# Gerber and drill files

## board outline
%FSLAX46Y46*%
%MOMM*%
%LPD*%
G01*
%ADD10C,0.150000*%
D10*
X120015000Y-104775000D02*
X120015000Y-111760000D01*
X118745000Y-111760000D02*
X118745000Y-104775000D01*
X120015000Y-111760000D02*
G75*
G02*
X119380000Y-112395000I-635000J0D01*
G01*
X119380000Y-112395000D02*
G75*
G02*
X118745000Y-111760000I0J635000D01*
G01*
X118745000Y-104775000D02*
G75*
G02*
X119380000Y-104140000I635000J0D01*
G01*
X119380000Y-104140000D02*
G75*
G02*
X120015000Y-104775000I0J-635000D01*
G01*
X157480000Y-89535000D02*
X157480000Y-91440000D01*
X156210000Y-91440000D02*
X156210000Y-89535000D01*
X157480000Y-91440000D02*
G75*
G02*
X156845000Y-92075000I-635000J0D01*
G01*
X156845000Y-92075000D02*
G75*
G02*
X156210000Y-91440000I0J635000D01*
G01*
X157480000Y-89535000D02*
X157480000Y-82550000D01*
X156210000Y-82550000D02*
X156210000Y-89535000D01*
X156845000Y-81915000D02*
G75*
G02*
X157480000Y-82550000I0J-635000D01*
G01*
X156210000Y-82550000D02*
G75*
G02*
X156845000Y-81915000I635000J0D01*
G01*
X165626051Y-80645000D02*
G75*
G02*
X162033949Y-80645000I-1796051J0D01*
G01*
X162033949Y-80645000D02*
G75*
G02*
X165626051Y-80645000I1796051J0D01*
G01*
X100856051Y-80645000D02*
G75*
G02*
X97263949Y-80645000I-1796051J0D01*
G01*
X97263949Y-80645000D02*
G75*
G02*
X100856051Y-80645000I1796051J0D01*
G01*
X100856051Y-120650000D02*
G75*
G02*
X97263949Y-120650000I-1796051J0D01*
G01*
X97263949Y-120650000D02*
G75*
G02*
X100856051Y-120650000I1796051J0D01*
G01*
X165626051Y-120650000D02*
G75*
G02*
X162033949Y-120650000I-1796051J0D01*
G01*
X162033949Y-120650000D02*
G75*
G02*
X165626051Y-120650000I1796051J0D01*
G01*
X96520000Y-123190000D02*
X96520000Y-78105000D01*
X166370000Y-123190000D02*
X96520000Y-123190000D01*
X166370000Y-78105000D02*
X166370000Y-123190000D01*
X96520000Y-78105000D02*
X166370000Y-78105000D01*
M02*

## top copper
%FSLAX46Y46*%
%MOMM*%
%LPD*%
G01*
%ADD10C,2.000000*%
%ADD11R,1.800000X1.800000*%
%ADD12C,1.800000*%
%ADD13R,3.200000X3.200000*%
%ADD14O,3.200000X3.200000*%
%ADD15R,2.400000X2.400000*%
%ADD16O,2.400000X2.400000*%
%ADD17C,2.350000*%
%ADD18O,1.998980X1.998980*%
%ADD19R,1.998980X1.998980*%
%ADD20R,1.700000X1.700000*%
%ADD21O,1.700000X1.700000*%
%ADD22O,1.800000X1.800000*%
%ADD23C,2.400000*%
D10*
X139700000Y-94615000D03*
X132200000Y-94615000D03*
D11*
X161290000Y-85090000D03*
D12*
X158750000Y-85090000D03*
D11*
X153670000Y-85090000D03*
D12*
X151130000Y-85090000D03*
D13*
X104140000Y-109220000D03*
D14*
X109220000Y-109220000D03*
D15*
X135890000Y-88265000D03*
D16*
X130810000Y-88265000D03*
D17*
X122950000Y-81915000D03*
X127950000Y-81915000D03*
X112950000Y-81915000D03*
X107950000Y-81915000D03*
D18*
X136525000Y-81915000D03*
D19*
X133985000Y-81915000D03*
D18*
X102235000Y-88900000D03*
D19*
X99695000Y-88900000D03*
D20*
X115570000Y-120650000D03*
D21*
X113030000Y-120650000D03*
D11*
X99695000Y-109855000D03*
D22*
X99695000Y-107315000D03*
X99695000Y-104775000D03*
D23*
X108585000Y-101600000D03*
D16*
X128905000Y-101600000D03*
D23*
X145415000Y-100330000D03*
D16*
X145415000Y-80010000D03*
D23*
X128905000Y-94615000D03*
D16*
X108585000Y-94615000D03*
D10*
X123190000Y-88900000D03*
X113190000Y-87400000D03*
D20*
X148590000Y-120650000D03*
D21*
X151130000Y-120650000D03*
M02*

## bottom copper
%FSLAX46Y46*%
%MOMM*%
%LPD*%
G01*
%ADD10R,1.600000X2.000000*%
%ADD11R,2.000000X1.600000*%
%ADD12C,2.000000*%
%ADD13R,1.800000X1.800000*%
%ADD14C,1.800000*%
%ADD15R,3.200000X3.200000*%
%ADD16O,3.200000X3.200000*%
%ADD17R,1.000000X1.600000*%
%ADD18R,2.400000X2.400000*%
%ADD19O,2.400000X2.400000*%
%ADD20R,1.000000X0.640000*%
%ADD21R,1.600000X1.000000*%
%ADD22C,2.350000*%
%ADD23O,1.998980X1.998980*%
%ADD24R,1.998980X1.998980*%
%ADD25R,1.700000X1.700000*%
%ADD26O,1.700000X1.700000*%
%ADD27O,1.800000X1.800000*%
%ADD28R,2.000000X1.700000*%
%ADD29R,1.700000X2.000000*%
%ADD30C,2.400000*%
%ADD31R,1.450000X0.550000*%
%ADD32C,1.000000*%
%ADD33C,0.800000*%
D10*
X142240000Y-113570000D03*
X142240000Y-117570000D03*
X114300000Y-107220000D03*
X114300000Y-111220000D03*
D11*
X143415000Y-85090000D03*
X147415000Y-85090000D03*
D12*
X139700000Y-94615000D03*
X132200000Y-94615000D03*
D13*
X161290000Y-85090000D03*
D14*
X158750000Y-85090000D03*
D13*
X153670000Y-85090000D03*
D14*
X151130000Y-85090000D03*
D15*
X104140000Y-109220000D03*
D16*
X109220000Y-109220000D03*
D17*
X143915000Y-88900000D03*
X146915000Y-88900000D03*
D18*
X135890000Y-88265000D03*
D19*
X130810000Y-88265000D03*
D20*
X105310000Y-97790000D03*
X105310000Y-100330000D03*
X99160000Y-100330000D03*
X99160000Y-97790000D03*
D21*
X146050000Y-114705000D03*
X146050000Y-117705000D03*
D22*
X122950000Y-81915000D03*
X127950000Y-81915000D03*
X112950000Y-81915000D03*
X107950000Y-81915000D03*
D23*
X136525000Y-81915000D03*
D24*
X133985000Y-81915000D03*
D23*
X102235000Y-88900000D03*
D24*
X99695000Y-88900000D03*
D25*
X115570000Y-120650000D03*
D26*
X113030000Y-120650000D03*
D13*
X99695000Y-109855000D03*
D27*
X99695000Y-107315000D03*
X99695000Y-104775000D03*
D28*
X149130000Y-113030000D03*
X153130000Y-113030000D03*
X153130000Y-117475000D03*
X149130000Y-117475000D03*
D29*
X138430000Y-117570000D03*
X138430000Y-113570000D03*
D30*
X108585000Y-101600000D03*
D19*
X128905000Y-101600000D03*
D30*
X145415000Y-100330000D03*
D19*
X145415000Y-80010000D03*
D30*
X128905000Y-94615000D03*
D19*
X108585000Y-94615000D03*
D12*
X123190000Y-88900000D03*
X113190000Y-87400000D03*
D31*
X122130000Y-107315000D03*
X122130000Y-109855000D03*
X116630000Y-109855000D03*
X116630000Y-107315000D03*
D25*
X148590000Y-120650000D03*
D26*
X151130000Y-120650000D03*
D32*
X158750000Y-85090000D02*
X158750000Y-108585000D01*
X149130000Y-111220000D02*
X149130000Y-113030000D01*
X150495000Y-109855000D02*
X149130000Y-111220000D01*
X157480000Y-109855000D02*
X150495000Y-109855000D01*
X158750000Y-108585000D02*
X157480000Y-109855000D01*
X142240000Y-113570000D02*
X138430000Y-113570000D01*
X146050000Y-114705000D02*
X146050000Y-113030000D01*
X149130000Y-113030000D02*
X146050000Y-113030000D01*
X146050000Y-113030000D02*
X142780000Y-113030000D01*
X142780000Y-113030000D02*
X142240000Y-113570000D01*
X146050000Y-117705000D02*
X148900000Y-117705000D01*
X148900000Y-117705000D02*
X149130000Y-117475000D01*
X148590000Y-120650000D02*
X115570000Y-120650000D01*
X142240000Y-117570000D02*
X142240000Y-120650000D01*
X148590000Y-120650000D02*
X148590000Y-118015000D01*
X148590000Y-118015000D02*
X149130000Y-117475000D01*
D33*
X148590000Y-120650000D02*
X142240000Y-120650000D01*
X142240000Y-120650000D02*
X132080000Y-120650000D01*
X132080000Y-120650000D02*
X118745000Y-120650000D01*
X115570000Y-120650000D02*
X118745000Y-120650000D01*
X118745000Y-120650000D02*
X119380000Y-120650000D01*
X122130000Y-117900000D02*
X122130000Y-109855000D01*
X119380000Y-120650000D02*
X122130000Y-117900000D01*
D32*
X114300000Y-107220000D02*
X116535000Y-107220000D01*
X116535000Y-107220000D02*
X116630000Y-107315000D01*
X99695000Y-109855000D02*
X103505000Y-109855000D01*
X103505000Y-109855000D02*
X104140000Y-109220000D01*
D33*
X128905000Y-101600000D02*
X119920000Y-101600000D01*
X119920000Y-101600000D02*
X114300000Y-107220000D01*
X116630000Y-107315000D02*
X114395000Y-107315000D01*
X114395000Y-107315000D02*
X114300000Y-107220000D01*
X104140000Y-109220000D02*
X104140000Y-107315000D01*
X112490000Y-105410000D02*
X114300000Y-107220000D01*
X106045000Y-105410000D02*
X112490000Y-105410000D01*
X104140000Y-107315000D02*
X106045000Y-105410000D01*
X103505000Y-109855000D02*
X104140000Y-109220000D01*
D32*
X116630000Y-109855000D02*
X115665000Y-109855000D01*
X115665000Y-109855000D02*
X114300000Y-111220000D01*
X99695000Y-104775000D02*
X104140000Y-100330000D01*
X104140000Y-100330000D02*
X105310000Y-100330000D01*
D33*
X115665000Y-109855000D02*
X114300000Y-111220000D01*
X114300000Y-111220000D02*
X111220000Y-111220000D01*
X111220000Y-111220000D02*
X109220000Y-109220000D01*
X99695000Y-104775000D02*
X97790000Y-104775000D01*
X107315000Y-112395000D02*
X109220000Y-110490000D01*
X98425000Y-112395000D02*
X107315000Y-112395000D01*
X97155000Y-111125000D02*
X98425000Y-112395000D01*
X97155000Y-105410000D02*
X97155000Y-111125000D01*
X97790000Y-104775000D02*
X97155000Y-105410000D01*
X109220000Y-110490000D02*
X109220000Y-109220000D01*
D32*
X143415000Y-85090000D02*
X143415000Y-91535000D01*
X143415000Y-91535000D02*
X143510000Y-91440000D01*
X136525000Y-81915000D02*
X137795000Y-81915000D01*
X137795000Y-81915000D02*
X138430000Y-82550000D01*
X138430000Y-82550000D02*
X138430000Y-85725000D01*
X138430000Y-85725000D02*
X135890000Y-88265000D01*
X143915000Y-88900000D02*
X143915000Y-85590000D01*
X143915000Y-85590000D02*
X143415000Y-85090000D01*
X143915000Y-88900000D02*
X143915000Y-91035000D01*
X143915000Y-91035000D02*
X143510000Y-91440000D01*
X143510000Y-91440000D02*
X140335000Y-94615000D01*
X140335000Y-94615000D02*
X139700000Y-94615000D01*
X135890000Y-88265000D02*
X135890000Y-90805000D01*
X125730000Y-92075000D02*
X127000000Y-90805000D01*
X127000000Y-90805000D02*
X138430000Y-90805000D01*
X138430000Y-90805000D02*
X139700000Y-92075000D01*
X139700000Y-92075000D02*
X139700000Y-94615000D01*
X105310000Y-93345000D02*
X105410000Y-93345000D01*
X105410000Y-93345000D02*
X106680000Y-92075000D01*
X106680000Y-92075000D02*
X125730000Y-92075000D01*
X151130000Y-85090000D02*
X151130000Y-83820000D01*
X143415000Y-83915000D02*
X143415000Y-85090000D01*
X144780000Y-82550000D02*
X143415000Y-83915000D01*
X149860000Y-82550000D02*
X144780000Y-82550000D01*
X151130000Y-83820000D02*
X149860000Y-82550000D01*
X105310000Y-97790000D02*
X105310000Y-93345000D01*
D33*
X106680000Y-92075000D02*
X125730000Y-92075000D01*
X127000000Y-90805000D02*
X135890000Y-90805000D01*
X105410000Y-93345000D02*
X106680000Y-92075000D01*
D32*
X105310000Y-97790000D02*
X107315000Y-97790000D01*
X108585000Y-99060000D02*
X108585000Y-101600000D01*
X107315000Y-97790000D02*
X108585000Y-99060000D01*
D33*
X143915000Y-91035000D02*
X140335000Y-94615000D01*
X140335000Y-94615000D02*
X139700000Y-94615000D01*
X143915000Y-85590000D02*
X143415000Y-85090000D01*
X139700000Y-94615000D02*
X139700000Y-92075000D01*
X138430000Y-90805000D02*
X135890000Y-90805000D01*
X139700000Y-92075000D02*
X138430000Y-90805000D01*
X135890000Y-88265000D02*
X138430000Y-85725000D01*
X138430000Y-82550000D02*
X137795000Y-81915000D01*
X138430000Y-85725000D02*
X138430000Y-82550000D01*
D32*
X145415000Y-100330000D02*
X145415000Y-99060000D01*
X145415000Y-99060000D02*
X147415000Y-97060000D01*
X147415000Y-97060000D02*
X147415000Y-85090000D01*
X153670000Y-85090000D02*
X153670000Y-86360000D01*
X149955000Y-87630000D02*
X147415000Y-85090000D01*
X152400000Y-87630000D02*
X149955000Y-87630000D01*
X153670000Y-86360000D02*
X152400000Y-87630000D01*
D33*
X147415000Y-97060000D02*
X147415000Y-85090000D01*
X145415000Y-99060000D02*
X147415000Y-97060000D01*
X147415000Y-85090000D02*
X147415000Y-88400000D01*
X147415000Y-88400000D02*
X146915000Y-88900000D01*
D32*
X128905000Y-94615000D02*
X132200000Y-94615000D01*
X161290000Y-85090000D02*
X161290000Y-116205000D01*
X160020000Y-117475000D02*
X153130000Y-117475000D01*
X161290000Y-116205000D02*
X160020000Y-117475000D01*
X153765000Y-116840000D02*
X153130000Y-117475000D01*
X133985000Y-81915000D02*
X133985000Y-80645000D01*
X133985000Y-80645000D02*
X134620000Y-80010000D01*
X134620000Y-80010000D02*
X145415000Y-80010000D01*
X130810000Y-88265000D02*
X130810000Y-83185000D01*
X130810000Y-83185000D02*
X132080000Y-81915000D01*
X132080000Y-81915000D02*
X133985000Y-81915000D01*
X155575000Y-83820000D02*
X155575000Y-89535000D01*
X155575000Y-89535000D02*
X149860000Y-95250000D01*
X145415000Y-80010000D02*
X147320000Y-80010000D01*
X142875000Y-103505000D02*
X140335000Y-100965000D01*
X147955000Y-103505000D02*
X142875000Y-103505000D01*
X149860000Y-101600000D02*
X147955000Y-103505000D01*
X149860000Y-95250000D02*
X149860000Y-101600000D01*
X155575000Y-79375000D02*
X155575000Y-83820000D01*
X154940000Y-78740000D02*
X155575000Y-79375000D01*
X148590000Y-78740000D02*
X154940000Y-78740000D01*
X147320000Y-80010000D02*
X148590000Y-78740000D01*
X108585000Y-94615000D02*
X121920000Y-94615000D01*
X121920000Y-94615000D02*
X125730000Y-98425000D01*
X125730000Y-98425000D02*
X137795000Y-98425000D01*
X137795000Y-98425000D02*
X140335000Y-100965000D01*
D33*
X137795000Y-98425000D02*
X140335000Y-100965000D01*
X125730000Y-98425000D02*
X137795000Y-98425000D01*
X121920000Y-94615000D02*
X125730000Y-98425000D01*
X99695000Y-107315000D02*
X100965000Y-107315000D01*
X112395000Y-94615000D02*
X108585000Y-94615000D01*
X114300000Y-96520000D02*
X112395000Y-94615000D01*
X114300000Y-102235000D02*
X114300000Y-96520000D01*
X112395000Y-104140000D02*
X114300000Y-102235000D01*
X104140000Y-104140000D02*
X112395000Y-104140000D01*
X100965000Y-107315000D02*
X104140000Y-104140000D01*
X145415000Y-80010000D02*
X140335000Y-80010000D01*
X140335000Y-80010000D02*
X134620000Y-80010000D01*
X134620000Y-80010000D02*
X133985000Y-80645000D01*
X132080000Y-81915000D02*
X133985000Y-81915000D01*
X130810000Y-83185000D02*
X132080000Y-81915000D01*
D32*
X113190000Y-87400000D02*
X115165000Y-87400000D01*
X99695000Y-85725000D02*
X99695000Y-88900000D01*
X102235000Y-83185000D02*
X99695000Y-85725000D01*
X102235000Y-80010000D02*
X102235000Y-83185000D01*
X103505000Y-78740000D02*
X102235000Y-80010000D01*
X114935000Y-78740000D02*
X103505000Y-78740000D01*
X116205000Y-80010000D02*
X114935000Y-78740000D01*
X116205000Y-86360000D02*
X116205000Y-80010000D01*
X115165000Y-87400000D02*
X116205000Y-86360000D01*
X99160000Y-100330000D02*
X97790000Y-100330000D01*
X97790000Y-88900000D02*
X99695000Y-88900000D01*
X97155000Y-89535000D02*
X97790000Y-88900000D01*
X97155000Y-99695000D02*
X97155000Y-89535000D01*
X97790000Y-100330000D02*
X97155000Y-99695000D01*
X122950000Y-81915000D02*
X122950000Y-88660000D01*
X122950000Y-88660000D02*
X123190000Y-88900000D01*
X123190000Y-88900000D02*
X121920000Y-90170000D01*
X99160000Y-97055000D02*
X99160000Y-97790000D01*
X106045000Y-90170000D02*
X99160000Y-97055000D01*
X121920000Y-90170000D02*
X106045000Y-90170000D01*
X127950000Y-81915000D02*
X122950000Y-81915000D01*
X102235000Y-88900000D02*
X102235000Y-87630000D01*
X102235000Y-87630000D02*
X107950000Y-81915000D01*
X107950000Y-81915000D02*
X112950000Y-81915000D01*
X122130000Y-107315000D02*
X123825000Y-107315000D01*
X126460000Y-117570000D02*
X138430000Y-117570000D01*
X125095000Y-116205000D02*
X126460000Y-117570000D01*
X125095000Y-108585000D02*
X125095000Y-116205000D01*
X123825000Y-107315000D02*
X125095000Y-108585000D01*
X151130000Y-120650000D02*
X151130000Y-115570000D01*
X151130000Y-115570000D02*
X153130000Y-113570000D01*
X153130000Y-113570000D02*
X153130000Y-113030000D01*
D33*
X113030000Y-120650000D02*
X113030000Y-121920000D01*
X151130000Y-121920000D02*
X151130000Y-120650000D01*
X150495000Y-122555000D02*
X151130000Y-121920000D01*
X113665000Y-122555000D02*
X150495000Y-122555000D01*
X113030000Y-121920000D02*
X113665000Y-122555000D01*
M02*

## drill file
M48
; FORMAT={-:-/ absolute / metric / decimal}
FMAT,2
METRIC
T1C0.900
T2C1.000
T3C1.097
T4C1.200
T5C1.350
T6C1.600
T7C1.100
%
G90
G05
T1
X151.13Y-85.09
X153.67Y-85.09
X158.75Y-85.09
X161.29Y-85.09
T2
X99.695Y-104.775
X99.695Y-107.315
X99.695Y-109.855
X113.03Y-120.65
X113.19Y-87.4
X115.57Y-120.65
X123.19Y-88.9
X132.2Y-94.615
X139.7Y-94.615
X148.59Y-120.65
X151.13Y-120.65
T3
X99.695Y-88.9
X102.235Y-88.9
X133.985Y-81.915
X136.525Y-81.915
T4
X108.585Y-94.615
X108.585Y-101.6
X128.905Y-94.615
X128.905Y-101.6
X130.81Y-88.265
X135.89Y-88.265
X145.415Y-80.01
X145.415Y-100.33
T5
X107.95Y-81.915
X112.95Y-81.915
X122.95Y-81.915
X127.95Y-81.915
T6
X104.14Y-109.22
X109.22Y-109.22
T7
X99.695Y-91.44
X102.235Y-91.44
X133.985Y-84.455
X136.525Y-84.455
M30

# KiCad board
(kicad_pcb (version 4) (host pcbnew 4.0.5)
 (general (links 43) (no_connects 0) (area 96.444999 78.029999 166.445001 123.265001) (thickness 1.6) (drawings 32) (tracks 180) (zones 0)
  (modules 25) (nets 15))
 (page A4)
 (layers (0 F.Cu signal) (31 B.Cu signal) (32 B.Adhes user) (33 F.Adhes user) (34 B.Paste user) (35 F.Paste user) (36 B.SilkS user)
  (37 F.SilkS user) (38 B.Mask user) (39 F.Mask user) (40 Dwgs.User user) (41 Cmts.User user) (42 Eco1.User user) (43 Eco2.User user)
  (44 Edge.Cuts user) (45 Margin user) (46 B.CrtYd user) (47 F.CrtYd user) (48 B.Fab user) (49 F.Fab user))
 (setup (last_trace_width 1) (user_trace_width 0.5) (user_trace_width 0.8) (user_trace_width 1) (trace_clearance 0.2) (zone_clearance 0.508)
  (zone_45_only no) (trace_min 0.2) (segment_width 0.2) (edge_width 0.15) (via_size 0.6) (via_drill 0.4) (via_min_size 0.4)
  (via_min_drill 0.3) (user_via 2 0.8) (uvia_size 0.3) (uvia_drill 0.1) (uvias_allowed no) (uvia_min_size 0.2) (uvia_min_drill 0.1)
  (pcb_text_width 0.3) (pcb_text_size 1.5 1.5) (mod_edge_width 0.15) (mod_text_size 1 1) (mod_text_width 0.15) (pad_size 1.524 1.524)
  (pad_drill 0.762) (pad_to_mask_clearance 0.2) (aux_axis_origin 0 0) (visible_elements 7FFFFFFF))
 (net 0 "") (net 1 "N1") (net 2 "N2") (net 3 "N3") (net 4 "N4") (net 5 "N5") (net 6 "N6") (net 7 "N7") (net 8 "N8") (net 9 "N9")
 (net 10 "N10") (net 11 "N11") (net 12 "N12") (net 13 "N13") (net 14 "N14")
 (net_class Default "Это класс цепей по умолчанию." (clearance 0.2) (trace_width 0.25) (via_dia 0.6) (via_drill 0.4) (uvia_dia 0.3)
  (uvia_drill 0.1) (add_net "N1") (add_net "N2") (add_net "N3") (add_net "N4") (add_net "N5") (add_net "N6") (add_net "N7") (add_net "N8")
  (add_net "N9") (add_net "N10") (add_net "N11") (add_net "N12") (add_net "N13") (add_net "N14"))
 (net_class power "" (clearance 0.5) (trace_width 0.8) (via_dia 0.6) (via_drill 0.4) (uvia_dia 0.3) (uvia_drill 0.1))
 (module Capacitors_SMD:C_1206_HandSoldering (layer B.Cu) (at 142.24 115.57 270)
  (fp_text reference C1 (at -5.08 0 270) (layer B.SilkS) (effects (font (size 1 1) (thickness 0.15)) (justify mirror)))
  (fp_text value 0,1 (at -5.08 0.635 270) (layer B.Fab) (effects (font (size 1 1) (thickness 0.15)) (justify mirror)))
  (pad 1 smd rect (at -2 0 270) (size 2 1.6) (layers B.Cu B.Paste B.Mask) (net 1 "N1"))
  (pad 2 smd rect (at 2 0 270) (size 2 1.6) (layers B.Cu B.Paste B.Mask) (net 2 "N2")))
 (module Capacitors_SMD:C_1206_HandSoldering (layer B.Cu) (at 114.3 109.22 270)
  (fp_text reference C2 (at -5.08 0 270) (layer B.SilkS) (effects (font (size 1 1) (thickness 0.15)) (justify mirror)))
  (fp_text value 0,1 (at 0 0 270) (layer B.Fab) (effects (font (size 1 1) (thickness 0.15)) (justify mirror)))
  (pad 1 smd rect (at -2 0 270) (size 2 1.6) (layers B.Cu B.Paste B.Mask) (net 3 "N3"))
  (pad 2 smd rect (at 2 0 270) (size 2 1.6) (layers B.Cu B.Paste B.Mask) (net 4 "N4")))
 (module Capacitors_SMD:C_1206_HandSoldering (layer B.Cu) (at 145.415 85.09)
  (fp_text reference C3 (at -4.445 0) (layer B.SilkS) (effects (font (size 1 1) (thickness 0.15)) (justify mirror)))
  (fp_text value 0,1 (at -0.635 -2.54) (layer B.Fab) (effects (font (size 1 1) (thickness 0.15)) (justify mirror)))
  (pad 1 smd rect (at -2 0) (size 2 1.6) (layers B.Cu B.Paste B.Mask) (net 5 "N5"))
  (pad 2 smd rect (at 2 0) (size 2 1.6) (layers B.Cu B.Paste B.Mask) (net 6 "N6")))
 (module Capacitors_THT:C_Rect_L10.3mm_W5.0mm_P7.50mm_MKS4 (layer F.Cu) (at 139.7 94.615 180)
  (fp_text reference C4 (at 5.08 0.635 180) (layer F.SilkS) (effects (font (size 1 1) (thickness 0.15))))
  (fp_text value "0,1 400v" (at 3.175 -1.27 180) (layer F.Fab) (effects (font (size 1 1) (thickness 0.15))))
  (pad 1 thru_hole circle (at 0 0 180) (size 2 2) (drill 1) (layers *.Cu *.Mask) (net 5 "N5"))
  (pad 2 thru_hole circle (at 7.5 0 180) (size 2 2) (drill 1) (layers *.Cu *.Mask) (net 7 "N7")))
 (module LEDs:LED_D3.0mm (layer F.Cu) (at 161.29 85.09 180)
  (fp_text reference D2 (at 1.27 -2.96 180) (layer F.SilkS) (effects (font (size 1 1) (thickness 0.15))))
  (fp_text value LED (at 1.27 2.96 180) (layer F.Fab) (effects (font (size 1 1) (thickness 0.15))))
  (pad 1 thru_hole rect (at 0 0 180) (size 1.8 1.8) (drill 0.9) (layers *.Cu *.Mask) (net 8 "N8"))
  (pad 2 thru_hole circle (at 2.54 0 180) (size 1.8 1.8) (drill 0.9) (layers *.Cu *.Mask) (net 1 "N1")))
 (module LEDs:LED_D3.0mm (layer F.Cu) (at 153.67 85.09 180)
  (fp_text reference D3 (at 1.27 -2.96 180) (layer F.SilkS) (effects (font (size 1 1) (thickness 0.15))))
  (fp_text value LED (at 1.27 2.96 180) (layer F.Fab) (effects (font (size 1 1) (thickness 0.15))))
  (pad 1 thru_hole rect (at 0 0 180) (size 1.8 1.8) (drill 0.9) (layers *.Cu *.Mask) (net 6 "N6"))
  (pad 2 thru_hole circle (at 2.54 0 180) (size 1.8 1.8) (drill 0.9) (layers *.Cu *.Mask) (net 5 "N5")))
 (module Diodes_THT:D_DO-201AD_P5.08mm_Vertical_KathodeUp (layer F.Cu) (at 104.14 109.22)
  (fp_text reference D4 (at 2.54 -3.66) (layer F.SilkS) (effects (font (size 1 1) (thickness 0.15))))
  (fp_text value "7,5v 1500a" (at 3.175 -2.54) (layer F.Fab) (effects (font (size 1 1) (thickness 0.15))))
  (pad 1 thru_hole rect (at 0 0) (size 3.2 3.2) (drill 1.6) (layers *.Cu *.Mask) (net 3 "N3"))
  (pad 2 thru_hole oval (at 5.08 0) (size 3.2 3.2) (drill 1.6) (layers *.Cu *.Mask) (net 4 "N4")))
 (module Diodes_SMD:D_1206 (layer B.Cu) (at 145.415 88.9)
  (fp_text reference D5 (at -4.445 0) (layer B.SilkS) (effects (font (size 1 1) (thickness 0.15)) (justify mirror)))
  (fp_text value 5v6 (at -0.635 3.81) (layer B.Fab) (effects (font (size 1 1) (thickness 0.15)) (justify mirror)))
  (pad 1 smd rect (at -1.5 0) (size 1 1.6) (layers B.Cu B.Paste B.Mask) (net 5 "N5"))
  (pad 2 smd rect (at 1.5 0) (size 1 1.6) (layers B.Cu B.Paste B.Mask) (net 6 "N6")))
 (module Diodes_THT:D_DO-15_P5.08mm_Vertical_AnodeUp (layer F.Cu) (at 135.89 88.265 180)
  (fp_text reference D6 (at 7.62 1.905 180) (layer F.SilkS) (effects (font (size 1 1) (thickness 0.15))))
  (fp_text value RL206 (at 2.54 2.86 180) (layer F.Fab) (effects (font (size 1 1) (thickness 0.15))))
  (pad 1 thru_hole rect (at 0 0 180) (size 2.4 2.4) (drill 1.2) (layers *.Cu *.Mask) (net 5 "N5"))
  (pad 2 thru_hole oval (at 5.08 0 180) (size 2.4 2.4) (drill 1.2) (layers *.Cu *.Mask) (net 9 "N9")))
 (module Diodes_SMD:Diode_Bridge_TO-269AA (layer B.Cu) (at 102.235 99.06 180)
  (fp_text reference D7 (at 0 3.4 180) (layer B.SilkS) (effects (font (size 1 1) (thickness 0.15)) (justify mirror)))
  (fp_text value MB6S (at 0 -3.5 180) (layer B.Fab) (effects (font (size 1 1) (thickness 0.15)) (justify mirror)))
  (pad 1 smd rect (at -3.075 1.27 180) (size 1 0.64) (layers B.Cu B.Paste B.Mask) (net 5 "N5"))
  (pad 2 smd rect (at -3.075 -1.27 180) (size 1 0.64) (layers B.Cu B.Paste B.Mask) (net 4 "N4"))
  (pad 3 smd rect (at 3.075 -1.27 180) (size 1 0.64) (layers B.Cu B.Paste B.Mask) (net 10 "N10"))
  (pad 4 smd rect (at 3.075 1.27 180) (size 1 0.64) (layers B.Cu B.Paste B.Mask) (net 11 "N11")))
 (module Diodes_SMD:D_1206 (layer B.Cu) (at 146.05 116.205 270)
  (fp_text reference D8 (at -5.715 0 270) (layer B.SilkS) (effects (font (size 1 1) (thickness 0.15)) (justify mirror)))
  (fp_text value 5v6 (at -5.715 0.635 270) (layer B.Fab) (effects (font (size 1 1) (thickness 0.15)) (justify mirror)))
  (pad 1 smd rect (at -1.5 0 270) (size 1 1.6) (layers B.Cu B.Paste B.Mask) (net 1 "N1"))
  (pad 2 smd rect (at 1.5 0 270) (size 1 1.6) (layers B.Cu B.Paste B.Mask) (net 2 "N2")))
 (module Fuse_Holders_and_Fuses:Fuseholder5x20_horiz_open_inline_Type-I (layer F.Cu) (at 107.95 81.915)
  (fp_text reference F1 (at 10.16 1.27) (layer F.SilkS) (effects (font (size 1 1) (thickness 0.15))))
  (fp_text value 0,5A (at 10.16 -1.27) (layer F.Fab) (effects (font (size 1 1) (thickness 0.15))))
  (pad 2 thru_hole circle (at 15 0) (size 2.35 2.35) (drill 1.35) (layers *.Cu *.Mask) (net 11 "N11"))
  (pad 2 thru_hole circle (at 20 0) (size 2.35 2.35) (drill 1.35) (layers *.Cu *.Mask) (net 11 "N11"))
  (pad 1 thru_hole circle (at 5 0) (size 2.35 2.35) (drill 1.35) (layers *.Cu *.Mask) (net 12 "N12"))
  (pad 1 thru_hole circle (at 0 0) (size 2.35 2.35) (drill 1.35) (layers *.Cu *.Mask) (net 12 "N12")))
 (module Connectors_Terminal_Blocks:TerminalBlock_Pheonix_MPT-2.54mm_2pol (layer F.Cu) (at 133.985 81.915)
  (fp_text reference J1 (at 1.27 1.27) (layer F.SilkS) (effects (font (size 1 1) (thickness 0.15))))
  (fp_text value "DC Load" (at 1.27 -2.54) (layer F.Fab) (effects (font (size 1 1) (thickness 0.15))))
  (pad 2 thru_hole oval (at 2.54 0) (size 1.99898 1.99898) (drill 1.09728) (layers *.Cu *.Mask) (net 5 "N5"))
  (pad 1 thru_hole rect (at 0 0) (size 1.99898 1.99898) (drill 1.09728) (layers *.Cu *.Mask) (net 9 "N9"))
  (pad "" np_thru_hole circle (at 0 2.54) (size 1.1 1.1) (drill 1.1) (layers *.Cu *.Mask))
  (pad "" np_thru_hole circle (at 2.54 2.54) (size 1.1 1.1) (drill 1.1) (layers *.Cu *.Mask)))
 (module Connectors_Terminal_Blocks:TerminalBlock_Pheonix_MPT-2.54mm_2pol (layer F.Cu) (at 99.695 88.9)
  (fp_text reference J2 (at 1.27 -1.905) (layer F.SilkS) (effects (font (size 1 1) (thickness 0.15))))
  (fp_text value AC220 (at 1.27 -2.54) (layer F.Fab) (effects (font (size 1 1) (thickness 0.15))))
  (pad 2 thru_hole oval (at 2.54 0) (size 1.99898 1.99898) (drill 1.09728) (layers *.Cu *.Mask) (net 12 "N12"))
  (pad 1 thru_hole rect (at 0 0) (size 1.99898 1.99898) (drill 1.09728) (layers *.Cu *.Mask) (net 10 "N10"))
  (pad "" np_thru_hole circle (at 0 2.54) (size 1.1 1.1) (drill 1.1) (layers *.Cu *.Mask))
  (pad "" np_thru_hole circle (at 2.54 2.54) (size 1.1 1.1) (drill 1.1) (layers *.Cu *.Mask)))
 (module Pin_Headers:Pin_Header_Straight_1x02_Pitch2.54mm (layer F.Cu) (at 115.57 120.65 270)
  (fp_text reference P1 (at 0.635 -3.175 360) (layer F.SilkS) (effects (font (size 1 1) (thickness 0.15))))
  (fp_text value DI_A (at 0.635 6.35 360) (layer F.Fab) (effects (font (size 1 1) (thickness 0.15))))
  (pad 1 thru_hole rect (at 0 0 270) (size 1.7 1.7) (drill 1) (layers *.Cu *.Mask) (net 2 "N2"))
  (pad 2 thru_hole oval (at 0 2.54 270) (size 1.7 1.7) (drill 1) (layers *.Cu *.Mask) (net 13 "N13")))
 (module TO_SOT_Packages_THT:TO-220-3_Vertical (layer F.Cu) (at 99.695 109.855 90)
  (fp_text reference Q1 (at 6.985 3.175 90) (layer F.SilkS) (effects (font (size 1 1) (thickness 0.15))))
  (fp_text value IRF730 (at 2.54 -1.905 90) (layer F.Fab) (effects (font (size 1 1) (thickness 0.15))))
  (pad 1 thru_hole rect (at 0 0 90) (size 1.8 1.8) (drill 1) (layers *.Cu *.Mask) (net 3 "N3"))
  (pad 2 thru_hole oval (at 2.54 0 90) (size 1.8 1.8) (drill 1) (layers *.Cu *.Mask) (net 9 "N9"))
  (pad 3 thru_hole oval (at 5.08 0 90) (size 1.8 1.8) (drill 1) (layers *.Cu *.Mask) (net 4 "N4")))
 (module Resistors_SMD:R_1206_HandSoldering (layer B.Cu) (at 151.13 113.03)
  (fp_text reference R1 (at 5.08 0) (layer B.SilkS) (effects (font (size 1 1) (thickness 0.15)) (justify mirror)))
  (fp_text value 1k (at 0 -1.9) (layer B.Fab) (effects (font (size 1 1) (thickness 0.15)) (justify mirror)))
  (pad 1 smd rect (at -2 0) (size 2 1.7) (layers B.Cu B.Paste B.Mask) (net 1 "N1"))
  (pad 2 smd rect (at 2 0) (size 2 1.7) (layers B.Cu B.Paste B.Mask) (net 13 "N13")))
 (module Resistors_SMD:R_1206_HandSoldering (layer B.Cu) (at 151.13 117.475 180)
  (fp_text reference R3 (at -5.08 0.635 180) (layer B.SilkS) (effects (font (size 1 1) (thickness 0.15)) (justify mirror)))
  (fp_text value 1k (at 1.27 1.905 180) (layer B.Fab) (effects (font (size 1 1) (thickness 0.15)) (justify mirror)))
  (pad 1 smd rect (at -2 0 180) (size 2 1.7) (layers B.Cu B.Paste B.Mask) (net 8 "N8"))
  (pad 2 smd rect (at 2 0 180) (size 2 1.7) (layers B.Cu B.Paste B.Mask) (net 2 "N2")))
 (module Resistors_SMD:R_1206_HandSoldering (layer B.Cu) (at 138.43 115.57 90)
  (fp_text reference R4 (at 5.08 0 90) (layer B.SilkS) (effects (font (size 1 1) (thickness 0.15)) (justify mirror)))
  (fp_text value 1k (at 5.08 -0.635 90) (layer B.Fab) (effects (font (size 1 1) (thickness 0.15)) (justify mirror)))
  (pad 1 smd rect (at -2 0 90) (size 2 1.7) (layers B.Cu B.Paste B.Mask) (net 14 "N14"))
  (pad 2 smd rect (at 2 0 90) (size 2 1.7) (layers B.Cu B.Paste B.Mask) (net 1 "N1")))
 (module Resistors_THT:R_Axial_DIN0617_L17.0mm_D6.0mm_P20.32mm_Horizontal (layer F.Cu) (at 108.585 101.6)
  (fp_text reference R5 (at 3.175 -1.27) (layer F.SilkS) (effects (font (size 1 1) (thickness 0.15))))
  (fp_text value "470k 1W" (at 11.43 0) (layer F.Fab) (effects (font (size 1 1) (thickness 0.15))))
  (pad 1 thru_hole circle (at 0 0) (size 2.4 2.4) (drill 1.2) (layers *.Cu *.Mask) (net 5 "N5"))
  (pad 2 thru_hole oval (at 20.32 0) (size 2.4 2.4) (drill 1.2) (layers *.Cu *.Mask) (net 3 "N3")))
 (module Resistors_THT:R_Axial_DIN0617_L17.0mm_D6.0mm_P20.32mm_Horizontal (layer F.Cu) (at 145.415 100.33 90)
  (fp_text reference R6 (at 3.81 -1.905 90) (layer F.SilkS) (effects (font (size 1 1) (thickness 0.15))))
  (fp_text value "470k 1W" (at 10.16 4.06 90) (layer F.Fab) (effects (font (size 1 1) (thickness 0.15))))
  (pad 1 thru_hole circle (at 0 0 90) (size 2.4 2.4) (drill 1.2) (layers *.Cu *.Mask) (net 6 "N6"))
  (pad 2 thru_hole oval (at 20.32 0 90) (size 2.4 2.4) (drill 1.2) (layers *.Cu *.Mask) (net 9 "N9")))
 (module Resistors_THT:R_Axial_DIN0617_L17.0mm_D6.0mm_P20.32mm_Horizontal (layer F.Cu) (at 128.905 94.615 180)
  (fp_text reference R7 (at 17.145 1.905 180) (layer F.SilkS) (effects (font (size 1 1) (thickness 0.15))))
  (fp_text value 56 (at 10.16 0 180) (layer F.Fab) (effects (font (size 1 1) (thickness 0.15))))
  (pad 1 thru_hole circle (at 0 0 180) (size 2.4 2.4) (drill 1.2) (layers *.Cu *.Mask) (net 7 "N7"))
  (pad 2 thru_hole oval (at 20.32 0 180) (size 2.4 2.4) (drill 1.2) (layers *.Cu *.Mask) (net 9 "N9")))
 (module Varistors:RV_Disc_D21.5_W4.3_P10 (layer F.Cu) (at 123.19 88.9 180)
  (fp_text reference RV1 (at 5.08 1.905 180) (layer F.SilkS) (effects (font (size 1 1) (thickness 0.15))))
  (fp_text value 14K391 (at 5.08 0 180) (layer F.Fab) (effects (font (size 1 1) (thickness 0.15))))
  (pad 1 thru_hole circle (at 0 0 180) (size 2 2) (drill 1) (layers *.Cu *.Mask) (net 11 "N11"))
  (pad 2 thru_hole circle (at 10 1.5 180) (size 2 2) (drill 1) (layers *.Cu *.Mask) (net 10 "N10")))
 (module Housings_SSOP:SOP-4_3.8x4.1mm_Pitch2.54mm (layer B.Cu) (at 119.38 108.585 180)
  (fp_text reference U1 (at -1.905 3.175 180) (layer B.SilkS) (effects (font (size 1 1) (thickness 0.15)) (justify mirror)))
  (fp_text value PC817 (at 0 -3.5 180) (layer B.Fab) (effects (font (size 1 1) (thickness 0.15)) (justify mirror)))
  (pad 1 smd rect (at -2.75 1.27 180) (size 1.45 0.55) (layers B.Cu B.Paste B.Mask) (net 14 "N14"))
  (pad 2 smd rect (at -2.75 -1.27 180) (size 1.45 0.55) (layers B.Cu B.Paste B.Mask) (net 2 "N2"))
  (pad 3 smd rect (at 2.75 -1.27 180) (size 1.45 0.55) (layers B.Cu B.Paste B.Mask) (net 4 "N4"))
  (pad 4 smd rect (at 2.75 1.27 180) (size 1.45 0.55) (layers B.Cu B.Paste B.Mask) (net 3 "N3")))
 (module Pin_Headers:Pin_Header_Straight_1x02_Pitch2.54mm (layer F.Cu) (at 148.59 120.65 90)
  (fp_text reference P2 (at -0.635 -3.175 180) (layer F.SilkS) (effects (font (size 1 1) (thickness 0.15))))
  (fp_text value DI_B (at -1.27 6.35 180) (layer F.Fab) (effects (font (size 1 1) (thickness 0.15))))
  (pad 1 thru_hole rect (at 0 0 90) (size 1.7 1.7) (drill 1) (layers *.Cu *.Mask) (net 2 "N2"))
  (pad 2 thru_hole oval (at 0 2.54 90) (size 1.7 1.7) (drill 1) (layers *.Cu *.Mask) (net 13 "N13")))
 (gr_line (start 120.015 104.775) (end 120.015 111.76) (angle 90) (layer Edge.Cuts) (width 0.15))
 (gr_line (start 118.745 111.76) (end 118.745 104.775) (angle 90) (layer Edge.Cuts) (width 0.15))
 (gr_arc (start 119.38 111.76) (end 120.015 111.76) (angle 90) (layer Edge.Cuts) (width 0.15))
 (gr_arc (start 119.38 111.76) (end 119.38 112.395) (angle 90) (layer Edge.Cuts) (width 0.15))
 (gr_arc (start 119.38 104.775) (end 118.745 104.775) (angle 90) (layer Edge.Cuts) (width 0.15))
 (gr_arc (start 119.38 104.775) (end 119.38 104.14) (angle 90) (layer Edge.Cuts) (width 0.15))
 (gr_line (start 157.48 89.535) (end 157.48 91.44) (angle 90) (layer Edge.Cuts) (width 0.15))
 (gr_line (start 156.21 91.44) (end 156.21 89.535) (angle 90) (layer Edge.Cuts) (width 0.15))
 (gr_arc (start 156.845 91.44) (end 157.48 91.44) (angle 90) (layer Edge.Cuts) (width 0.15))
 (gr_arc (start 156.845 91.44) (end 156.845 92.075) (angle 90) (layer Edge.Cuts) (width 0.15))
 (gr_line (start 157.48 89.535) (end 157.48 82.55) (angle 90) (layer Edge.Cuts) (width 0.15))
 (gr_line (start 156.21 82.55) (end 156.21 89.535) (angle 90) (layer Edge.Cuts) (width 0.15))
 (gr_arc (start 156.845 82.55) (end 156.845 81.915) (angle 90) (layer Edge.Cuts) (width 0.15))
 (gr_arc (start 156.845 82.55) (end 156.21 82.55) (angle 90) (layer Edge.Cuts) (width 0.15))
 (gr_circle (center 163.83 80.645) (end 165.1 79.375) (layer Edge.Cuts) (width 0.15))
 (gr_circle (center 99.06 80.645) (end 97.79 79.375) (layer Edge.Cuts) (width 0.15))
 (gr_circle (center 99.06 120.65) (end 97.79 121.92) (layer Edge.Cuts) (width 0.15))
 (gr_circle (center 163.83 120.65) (end 165.1 121.92) (layer Edge.Cuts) (width 0.15))
 (gr_line (start 96.52 123.19) (end 96.52 78.105) (angle 90) (layer Edge.Cuts) (width 0.15))
 (gr_line (start 166.37 123.19) (end 96.52 123.19) (angle 90) (layer Edge.Cuts) (width 0.15))
 (gr_line (start 166.37 78.105) (end 166.37 123.19) (angle 90) (layer Edge.Cuts) (width 0.15))
 (gr_line (start 96.52 78.105) (end 166.37 78.105) (angle 90) (layer Edge.Cuts) (width 0.15))
 (segment (start 158.75 85.09) (end 158.75 108.585) (width 1) (layer B.Cu) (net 1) (status 400000))
 (segment (start 149.13 111.22) (end 149.13 113.03) (width 1) (layer B.Cu) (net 1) (status 800000))
 (segment (start 150.495 109.855) (end 149.13 111.22) (width 1) (layer B.Cu) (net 1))
 (segment (start 157.48 109.855) (end 150.495 109.855) (width 1) (layer B.Cu) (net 1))
 (segment (start 158.75 108.585) (end 157.48 109.855) (width 1) (layer B.Cu) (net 1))
 (segment (start 142.24 113.57) (end 138.43 113.57) (width 1) (layer B.Cu) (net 1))
 (segment (start 146.05 114.705) (end 146.05 113.03) (width 1) (layer B.Cu) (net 1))
 (segment (start 149.13 113.03) (end 146.05 113.03) (width 1) (layer B.Cu) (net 1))
 (segment (start 146.05 113.03) (end 142.78 113.03) (width 1) (layer B.Cu) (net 1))
 (segment (start 142.78 113.03) (end 142.24 113.57) (width 1) (layer B.Cu) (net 1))
 (segment (start 146.05 117.705) (end 148.9 117.705) (width 1) (layer B.Cu) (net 2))
 (segment (start 148.9 117.705) (end 149.13 117.475) (width 1) (layer B.Cu) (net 2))
 (segment (start 148.59 120.65) (end 115.57 120.65) (width 1) (layer B.Cu) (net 2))
 (segment (start 142.24 117.57) (end 142.24 120.65) (width 1) (layer B.Cu) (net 2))
 (segment (start 148.59 120.65) (end 148.59 118.015) (width 1) (layer B.Cu) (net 2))
 (segment (start 148.59 118.015) (end 149.13 117.475) (width 1) (layer B.Cu) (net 2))
 (segment (start 148.59 120.65) (end 142.24 120.65) (width 0.8) (layer B.Cu) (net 2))
 (segment (start 142.24 120.65) (end 132.08 120.65) (width 0.8) (layer B.Cu) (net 2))
 (segment (start 132.08 120.65) (end 118.745 120.65) (width 0.8) (layer B.Cu) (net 2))
 (segment (start 115.57 120.65) (end 118.745 120.65) (width 0.8) (layer B.Cu) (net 2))
 (segment (start 118.745 120.65) (end 119.38 120.65) (width 0.8) (layer B.Cu) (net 2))
 (segment (start 122.13 117.9) (end 122.13 109.855) (width 0.8) (layer B.Cu) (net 2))
 (segment (start 119.38 120.65) (end 122.13 117.9) (width 0.8) (layer B.Cu) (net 2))
 (segment (start 114.3 107.22) (end 116.535 107.22) (width 1) (layer B.Cu) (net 3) (status C00000))
 (segment (start 116.535 107.22) (end 116.63 107.315) (width 1) (layer B.Cu) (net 3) (status C00000))
 (segment (start 99.695 109.855) (end 103.505 109.855) (width 1) (layer B.Cu) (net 3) (status C00000))
 (segment (start 103.505 109.855) (end 104.14 109.22) (width 1) (layer B.Cu) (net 3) (status C00000))
 (segment (start 128.905 101.6) (end 119.92 101.6) (width 0.8) (layer B.Cu) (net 3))
 (segment (start 119.92 101.6) (end 114.3 107.22) (width 0.8) (layer B.Cu) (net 3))
 (segment (start 116.63 107.315) (end 114.395 107.315) (width 0.8) (layer B.Cu) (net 3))
 (segment (start 114.395 107.315) (end 114.3 107.22) (width 0.8) (layer B.Cu) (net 3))
 (segment (start 104.14 109.22) (end 104.14 107.315) (width 0.8) (layer B.Cu) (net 3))
 (segment (start 112.49 105.41) (end 114.3 107.22) (width 0.8) (layer B.Cu) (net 3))
 (segment (start 106.045 105.41) (end 112.49 105.41) (width 0.8) (layer B.Cu) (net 3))
 (segment (start 104.14 107.315) (end 106.045 105.41) (width 0.8) (layer B.Cu) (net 3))
 (segment (start 103.505 109.855) (end 104.14 109.22) (width 0.8) (layer B.Cu) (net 3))
 (segment (start 116.63 109.855) (end 115.665 109.855) (width 1) (layer B.Cu) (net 4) (status 400000))
 (segment (start 115.665 109.855) (end 114.3 111.22) (width 1) (layer B.Cu) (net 4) (status 800000))
 (segment (start 99.695 104.775) (end 104.14 100.33) (width 1) (layer B.Cu) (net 4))
 (segment (start 104.14 100.33) (end 105.31 100.33) (width 1) (layer B.Cu) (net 4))
 (segment (start 115.665 109.855) (end 114.3 111.22) (width 0.8) (layer B.Cu) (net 4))
 (segment (start 114.3 111.22) (end 111.22 111.22) (width 0.8) (layer B.Cu) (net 4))
 (segment (start 111.22 111.22) (end 109.22 109.22) (width 0.8) (layer B.Cu) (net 4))
 (segment (start 99.695 104.775) (end 97.79 104.775) (width 0.8) (layer B.Cu) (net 4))
 (segment (start 107.315 112.395) (end 109.22 110.49) (width 0.8) (layer B.Cu) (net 4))
 (segment (start 98.425 112.395) (end 107.315 112.395) (width 0.8) (layer B.Cu) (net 4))
 (segment (start 97.155 111.125) (end 98.425 112.395) (width 0.8) (layer B.Cu) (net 4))
 (segment (start 97.155 105.41) (end 97.155 111.125) (width 0.8) (layer B.Cu) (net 4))
 (segment (start 97.79 104.775) (end 97.155 105.41) (width 0.8) (layer B.Cu) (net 4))
 (segment (start 109.22 110.49) (end 109.22 109.22) (width 0.8) (layer B.Cu) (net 4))
 (segment (start 143.415 85.09) (end 143.415 91.535) (width 1) (layer B.Cu) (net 5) (status 400000))
 (segment (start 143.415 91.535) (end 143.51 91.44) (width 1) (layer B.Cu) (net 5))
 (segment (start 136.525 81.915) (end 137.795 81.915) (width 1) (layer B.Cu) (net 5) (status 400000))
 (segment (start 137.795 81.915) (end 138.43 82.55) (width 1) (layer B.Cu) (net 5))
 (segment (start 138.43 82.55) (end 138.43 85.725) (width 1) (layer B.Cu) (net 5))
 (segment (start 138.43 85.725) (end 135.89 88.265) (width 1) (layer B.Cu) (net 5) (status 800000))
 (segment (start 143.915 88.9) (end 143.915 85.59) (width 1) (layer B.Cu) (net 5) (status C00000))
 (segment (start 143.915 85.59) (end 143.415 85.09) (width 1) (layer B.Cu) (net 5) (status C00000))
 (segment (start 143.915 88.9) (end 143.915 91.035) (width 1) (layer B.Cu) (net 5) (status 400000))
 (segment (start 143.915 91.035) (end 143.51 91.44) (width 1) (layer B.Cu) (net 5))
 (segment (start 143.51 91.44) (end 140.335 94.615) (width 1) (layer B.Cu) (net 5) (status 800000))
 (segment (start 140.335 94.615) (end 139.7 94.615) (width 1) (layer B.Cu) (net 5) (status C00000))
 (segment (start 135.89 88.265) (end 135.89 90.805) (width 1) (layer B.Cu) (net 5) (status 400000))
 (segment (start 125.73 92.075) (end 127 90.805) (width 1) (layer B.Cu) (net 5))
 (segment (start 127 90.805) (end 138.43 90.805) (width 1) (layer B.Cu) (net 5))
 (segment (start 138.43 90.805) (end 139.7 92.075) (width 1) (layer B.Cu) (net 5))
 (segment (start 139.7 92.075) (end 139.7 94.615) (width 1) (layer B.Cu) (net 5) (status 800000))
 (segment (start 105.31 93.345) (end 105.41 93.345) (width 1) (layer B.Cu) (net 5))
 (segment (start 105.41 93.345) (end 106.68 92.075) (width 1) (layer B.Cu) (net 5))
 (segment (start 106.68 92.075) (end 125.73 92.075) (width 1) (layer B.Cu) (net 5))
 (segment (start 151.13 85.09) (end 151.13 83.82) (width 1) (layer B.Cu) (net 5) (status 400000))
 (segment (start 143.415 83.915) (end 143.415 85.09) (width 1) (layer B.Cu) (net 5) (status 800000))
 (segment (start 144.78 82.55) (end 143.415 83.915) (width 1) (layer B.Cu) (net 5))
 (segment (start 149.86 82.55) (end 144.78 82.55) (width 1) (layer B.Cu) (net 5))
 (segment (start 151.13 83.82) (end 149.86 82.55) (width 1) (layer B.Cu) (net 5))
 (segment (start 105.31 97.79) (end 105.31 93.345) (width 1) (layer B.Cu) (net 5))
 (segment (start 106.68 92.075) (end 125.73 92.075) (width 0.8) (layer B.Cu) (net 5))
 (segment (start 127 90.805) (end 135.89 90.805) (width 0.8) (layer B.Cu) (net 5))
 (segment (start 105.41 93.345) (end 106.68 92.075) (width 0.8) (layer B.Cu) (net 5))
 (segment (start 105.31 97.79) (end 107.315 97.79) (width 1) (layer B.Cu) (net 5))
 (segment (start 108.585 99.06) (end 108.585 101.6) (width 1) (layer B.Cu) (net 5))
 (segment (start 107.315 97.79) (end 108.585 99.06) (width 1) (layer B.Cu) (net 5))
 (segment (start 143.915 91.035) (end 140.335 94.615) (width 0.8) (layer B.Cu) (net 5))
 (segment (start 140.335 94.615) (end 139.7 94.615) (width 0.8) (layer B.Cu) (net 5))
 (segment (start 143.915 85.59) (end 143.415 85.09) (width 0.8) (layer B.Cu) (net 5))
 (segment (start 139.7 94.615) (end 139.7 92.075) (width 0.8) (layer B.Cu) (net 5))
 (segment (start 138.43 90.805) (end 135.89 90.805) (width 0.8) (layer B.Cu) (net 5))
 (segment (start 139.7 92.075) (end 138.43 90.805) (width 0.8) (layer B.Cu) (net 5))
 (segment (start 135.89 88.265) (end 138.43 85.725) (width 0.8) (layer B.Cu) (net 5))
 (segment (start 138.43 82.55) (end 137.795 81.915) (width 0.8) (layer B.Cu) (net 5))
 (segment (start 138.43 85.725) (end 138.43 82.55) (width 0.8) (layer B.Cu) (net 5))
 (segment (start 145.415 100.33) (end 145.415 99.06) (width 1) (layer B.Cu) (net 6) (status 400000))
 (segment (start 145.415 99.06) (end 147.415 97.06) (width 1) (layer B.Cu) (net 6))
 (segment (start 147.415 97.06) (end 147.415 85.09) (width 1) (layer B.Cu) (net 6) (status 800000))
 (segment (start 153.67 85.09) (end 153.67 86.36) (width 1) (layer B.Cu) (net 6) (status 400000))
 (segment (start 149.955 87.63) (end 147.415 85.09) (width 1) (layer B.Cu) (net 6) (status 800000))
 (segment (start 152.4 87.63) (end 149.955 87.63) (width 1) (layer B.Cu) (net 6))
 (segment (start 153.67 86.36) (end 152.4 87.63) (width 1) (layer B.Cu) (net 6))
 (segment (start 147.415 97.06) (end 147.415 85.09) (width 0.8) (layer B.Cu) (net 6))
 (segment (start 145.415 99.06) (end 147.415 97.06) (width 0.8) (layer B.Cu) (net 6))
 (segment (start 147.415 85.09) (end 147.415 88.4) (width 0.8) (layer B.Cu) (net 6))
 (segment (start 147.415 88.4) (end 146.915 88.9) (width 0.8) (layer B.Cu) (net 6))
 (segment (start 128.905 94.615) (end 132.2 94.615) (width 1) (layer B.Cu) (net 7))
 (segment (start 161.29 85.09) (end 161.29 116.205) (width 1) (layer B.Cu) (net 8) (status 400000))
 (segment (start 160.02 117.475) (end 153.13 117.475) (width 1) (layer B.Cu) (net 8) (status 800000))
 (segment (start 161.29 116.205) (end 160.02 117.475) (width 1) (layer B.Cu) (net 8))
 (segment (start 153.765 116.84) (end 153.13 117.475) (width 1) (layer B.Cu) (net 8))
 (segment (start 133.985 81.915) (end 133.985 80.645) (width 1) (layer B.Cu) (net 9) (status 400000))
 (segment (start 133.985 80.645) (end 134.62 80.01) (width 1) (layer B.Cu) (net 9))
 (segment (start 134.62 80.01) (end 145.415 80.01) (width 1) (layer B.Cu) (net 9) (status 800000))
 (segment (start 130.81 88.265) (end 130.81 83.185) (width 1) (layer B.Cu) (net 9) (status 400000))
 (segment (start 130.81 83.185) (end 132.08 81.915) (width 1) (layer B.Cu) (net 9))
 (segment (start 132.08 81.915) (end 133.985 81.915) (width 1) (layer B.Cu) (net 9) (status 800000))
 (segment (start 155.575 83.82) (end 155.575 89.535) (width 1) (layer B.Cu) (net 9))
 (segment (start 155.575 89.535) (end 149.86 95.25) (width 1) (layer B.Cu) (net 9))
 (segment (start 145.415 80.01) (end 147.32 80.01) (width 1) (layer B.Cu) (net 9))
 (segment (start 142.875 103.505) (end 140.335 100.965) (width 1) (layer B.Cu) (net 9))
 (segment (start 147.955 103.505) (end 142.875 103.505) (width 1) (layer B.Cu) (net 9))
 (segment (start 149.86 101.6) (end 147.955 103.505) (width 1) (layer B.Cu) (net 9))
 (segment (start 149.86 95.25) (end 149.86 101.6) (width 1) (layer B.Cu) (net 9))
 (segment (start 155.575 79.375) (end 155.575 83.82) (width 1) (layer B.Cu) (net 9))
 (segment (start 154.94 78.74) (end 155.575 79.375) (width 1) (layer B.Cu) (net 9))
 (segment (start 148.59 78.74) (end 154.94 78.74) (width 1) (layer B.Cu) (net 9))
 (segment (start 147.32 80.01) (end 148.59 78.74) (width 1) (layer B.Cu) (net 9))
 (segment (start 108.585 94.615) (end 121.92 94.615) (width 1) (layer B.Cu) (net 9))
 (segment (start 121.92 94.615) (end 125.73 98.425) (width 1) (layer B.Cu) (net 9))
 (segment (start 125.73 98.425) (end 137.795 98.425) (width 1) (layer B.Cu) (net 9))
 (segment (start 137.795 98.425) (end 140.335 100.965) (width 1) (layer B.Cu) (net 9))
 (segment (start 137.795 98.425) (end 140.335 100.965) (width 0.8) (layer B.Cu) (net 9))
 (segment (start 125.73 98.425) (end 137.795 98.425) (width 0.8) (layer B.Cu) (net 9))
 (segment (start 121.92 94.615) (end 125.73 98.425) (width 0.8) (layer B.Cu) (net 9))
 (segment (start 99.695 107.315) (end 100.965 107.315) (width 0.8) (layer B.Cu) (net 9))
 (segment (start 112.395 94.615) (end 108.585 94.615) (width 0.8) (layer B.Cu) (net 9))
 (segment (start 114.3 96.52) (end 112.395 94.615) (width 0.8) (layer B.Cu) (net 9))
 (segment (start 114.3 102.235) (end 114.3 96.52) (width 0.8) (layer B.Cu) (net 9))
 (segment (start 112.395 104.14) (end 114.3 102.235) (width 0.8) (layer B.Cu) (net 9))
 (segment (start 104.14 104.14) (end 112.395 104.14) (width 0.8) (layer B.Cu) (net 9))
 (segment (start 100.965 107.315) (end 104.14 104.14) (width 0.8) (layer B.Cu) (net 9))
 (segment (start 145.415 80.01) (end 140.335 80.01) (width 0.8) (layer B.Cu) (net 9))
 (segment (start 140.335 80.01) (end 134.62 80.01) (width 0.8) (layer B.Cu) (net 9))
 (segment (start 134.62 80.01) (end 133.985 80.645) (width 0.8) (layer B.Cu) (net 9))
 (segment (start 132.08 81.915) (end 133.985 81.915) (width 0.8) (layer B.Cu) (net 9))
 (segment (start 130.81 83.185) (end 132.08 81.915) (width 0.8) (layer B.Cu) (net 9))
 (segment (start 113.19 87.4) (end 115.165 87.4) (width 1) (layer B.Cu) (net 10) (status 400000))
 (segment (start 99.695 85.725) (end 99.695 88.9) (width 1) (layer B.Cu) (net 10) (status 800000))
 (segment (start 102.235 83.185) (end 99.695 85.725) (width 1) (layer B.Cu) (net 10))
 (segment (start 102.235 80.01) (end 102.235 83.185) (width 1) (layer B.Cu) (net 10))
 (segment (start 103.505 78.74) (end 102.235 80.01) (width 1) (layer B.Cu) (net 10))
 (segment (start 114.935 78.74) (end 103.505 78.74) (width 1) (layer B.Cu) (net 10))
 (segment (start 116.205 80.01) (end 114.935 78.74) (width 1) (layer B.Cu) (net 10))
 (segment (start 116.205 86.36) (end 116.205 80.01) (width 1) (layer B.Cu) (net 10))
 (segment (start 115.165 87.4) (end 116.205 86.36) (width 1) (layer B.Cu) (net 10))
 (segment (start 99.16 100.33) (end 97.79 100.33) (width 1) (layer B.Cu) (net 10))
 (segment (start 97.79 88.9) (end 99.695 88.9) (width 1) (layer B.Cu) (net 10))
 (segment (start 97.155 89.535) (end 97.79 88.9) (width 1) (layer B.Cu) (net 10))
 (segment (start 97.155 99.695) (end 97.155 89.535) (width 1) (layer B.Cu) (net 10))
 (segment (start 97.79 100.33) (end 97.155 99.695) (width 1) (layer B.Cu) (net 10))
 (segment (start 122.95 81.915) (end 122.95 88.66) (width 1) (layer B.Cu) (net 11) (status C00000))
 (segment (start 122.95 88.66) (end 123.19 88.9) (width 1) (layer B.Cu) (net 11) (status C00000))
 (segment (start 123.19 88.9) (end 121.92 90.17) (width 1) (layer B.Cu) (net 11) (status 400000))
 (segment (start 99.16 97.055) (end 99.16 97.79) (width 1) (layer B.Cu) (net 11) (status 800000))
 (segment (start 106.045 90.17) (end 99.16 97.055) (width 1) (layer B.Cu) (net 11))
 (segment (start 121.92 90.17) (end 106.045 90.17) (width 1) (layer B.Cu) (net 11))
 (segment (start 127.95 81.915) (end 122.95 81.915) (width 1) (layer B.Cu) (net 11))
 (segment (start 102.235 88.9) (end 102.235 87.63) (width 1) (layer B.Cu) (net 12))
 (segment (start 102.235 87.63) (end 107.95 81.915) (width 1) (layer B.Cu) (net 12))
 (segment (start 107.95 81.915) (end 112.95 81.915) (width 1) (layer B.Cu) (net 12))
 (segment (start 122.13 107.315) (end 123.825 107.315) (width 1) (layer B.Cu) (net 14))
 (segment (start 126.46 117.57) (end 138.43 117.57) (width 1) (layer B.Cu) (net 14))
 (segment (start 125.095 116.205) (end 126.46 117.57) (width 1) (layer B.Cu) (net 14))
 (segment (start 125.095 108.585) (end 125.095 116.205) (width 1) (layer B.Cu) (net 14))
 (segment (start 123.825 107.315) (end 125.095 108.585) (width 1) (layer B.Cu) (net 14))
 (segment (start 151.13 120.65) (end 151.13 115.57) (width 1) (layer B.Cu) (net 13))
 (segment (start 151.13 115.57) (end 153.13 113.57) (width 1) (layer B.Cu) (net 13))
 (segment (start 153.13 113.57) (end 153.13 113.03) (width 1) (layer B.Cu) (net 13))
 (segment (start 113.03 120.65) (end 113.03 121.92) (width 0.8) (layer B.Cu) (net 13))
 (segment (start 151.13 121.92) (end 151.13 120.65) (width 0.8) (layer B.Cu) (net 13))
 (segment (start 150.495 122.555) (end 151.13 121.92) (width 0.8) (layer B.Cu) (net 13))
 (segment (start 113.665 122.555) (end 150.495 122.555) (width 0.8) (layer B.Cu) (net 13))
 (segment (start 113.03 121.92) (end 113.665 122.555) (width 0.8) (layer B.Cu) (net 13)))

